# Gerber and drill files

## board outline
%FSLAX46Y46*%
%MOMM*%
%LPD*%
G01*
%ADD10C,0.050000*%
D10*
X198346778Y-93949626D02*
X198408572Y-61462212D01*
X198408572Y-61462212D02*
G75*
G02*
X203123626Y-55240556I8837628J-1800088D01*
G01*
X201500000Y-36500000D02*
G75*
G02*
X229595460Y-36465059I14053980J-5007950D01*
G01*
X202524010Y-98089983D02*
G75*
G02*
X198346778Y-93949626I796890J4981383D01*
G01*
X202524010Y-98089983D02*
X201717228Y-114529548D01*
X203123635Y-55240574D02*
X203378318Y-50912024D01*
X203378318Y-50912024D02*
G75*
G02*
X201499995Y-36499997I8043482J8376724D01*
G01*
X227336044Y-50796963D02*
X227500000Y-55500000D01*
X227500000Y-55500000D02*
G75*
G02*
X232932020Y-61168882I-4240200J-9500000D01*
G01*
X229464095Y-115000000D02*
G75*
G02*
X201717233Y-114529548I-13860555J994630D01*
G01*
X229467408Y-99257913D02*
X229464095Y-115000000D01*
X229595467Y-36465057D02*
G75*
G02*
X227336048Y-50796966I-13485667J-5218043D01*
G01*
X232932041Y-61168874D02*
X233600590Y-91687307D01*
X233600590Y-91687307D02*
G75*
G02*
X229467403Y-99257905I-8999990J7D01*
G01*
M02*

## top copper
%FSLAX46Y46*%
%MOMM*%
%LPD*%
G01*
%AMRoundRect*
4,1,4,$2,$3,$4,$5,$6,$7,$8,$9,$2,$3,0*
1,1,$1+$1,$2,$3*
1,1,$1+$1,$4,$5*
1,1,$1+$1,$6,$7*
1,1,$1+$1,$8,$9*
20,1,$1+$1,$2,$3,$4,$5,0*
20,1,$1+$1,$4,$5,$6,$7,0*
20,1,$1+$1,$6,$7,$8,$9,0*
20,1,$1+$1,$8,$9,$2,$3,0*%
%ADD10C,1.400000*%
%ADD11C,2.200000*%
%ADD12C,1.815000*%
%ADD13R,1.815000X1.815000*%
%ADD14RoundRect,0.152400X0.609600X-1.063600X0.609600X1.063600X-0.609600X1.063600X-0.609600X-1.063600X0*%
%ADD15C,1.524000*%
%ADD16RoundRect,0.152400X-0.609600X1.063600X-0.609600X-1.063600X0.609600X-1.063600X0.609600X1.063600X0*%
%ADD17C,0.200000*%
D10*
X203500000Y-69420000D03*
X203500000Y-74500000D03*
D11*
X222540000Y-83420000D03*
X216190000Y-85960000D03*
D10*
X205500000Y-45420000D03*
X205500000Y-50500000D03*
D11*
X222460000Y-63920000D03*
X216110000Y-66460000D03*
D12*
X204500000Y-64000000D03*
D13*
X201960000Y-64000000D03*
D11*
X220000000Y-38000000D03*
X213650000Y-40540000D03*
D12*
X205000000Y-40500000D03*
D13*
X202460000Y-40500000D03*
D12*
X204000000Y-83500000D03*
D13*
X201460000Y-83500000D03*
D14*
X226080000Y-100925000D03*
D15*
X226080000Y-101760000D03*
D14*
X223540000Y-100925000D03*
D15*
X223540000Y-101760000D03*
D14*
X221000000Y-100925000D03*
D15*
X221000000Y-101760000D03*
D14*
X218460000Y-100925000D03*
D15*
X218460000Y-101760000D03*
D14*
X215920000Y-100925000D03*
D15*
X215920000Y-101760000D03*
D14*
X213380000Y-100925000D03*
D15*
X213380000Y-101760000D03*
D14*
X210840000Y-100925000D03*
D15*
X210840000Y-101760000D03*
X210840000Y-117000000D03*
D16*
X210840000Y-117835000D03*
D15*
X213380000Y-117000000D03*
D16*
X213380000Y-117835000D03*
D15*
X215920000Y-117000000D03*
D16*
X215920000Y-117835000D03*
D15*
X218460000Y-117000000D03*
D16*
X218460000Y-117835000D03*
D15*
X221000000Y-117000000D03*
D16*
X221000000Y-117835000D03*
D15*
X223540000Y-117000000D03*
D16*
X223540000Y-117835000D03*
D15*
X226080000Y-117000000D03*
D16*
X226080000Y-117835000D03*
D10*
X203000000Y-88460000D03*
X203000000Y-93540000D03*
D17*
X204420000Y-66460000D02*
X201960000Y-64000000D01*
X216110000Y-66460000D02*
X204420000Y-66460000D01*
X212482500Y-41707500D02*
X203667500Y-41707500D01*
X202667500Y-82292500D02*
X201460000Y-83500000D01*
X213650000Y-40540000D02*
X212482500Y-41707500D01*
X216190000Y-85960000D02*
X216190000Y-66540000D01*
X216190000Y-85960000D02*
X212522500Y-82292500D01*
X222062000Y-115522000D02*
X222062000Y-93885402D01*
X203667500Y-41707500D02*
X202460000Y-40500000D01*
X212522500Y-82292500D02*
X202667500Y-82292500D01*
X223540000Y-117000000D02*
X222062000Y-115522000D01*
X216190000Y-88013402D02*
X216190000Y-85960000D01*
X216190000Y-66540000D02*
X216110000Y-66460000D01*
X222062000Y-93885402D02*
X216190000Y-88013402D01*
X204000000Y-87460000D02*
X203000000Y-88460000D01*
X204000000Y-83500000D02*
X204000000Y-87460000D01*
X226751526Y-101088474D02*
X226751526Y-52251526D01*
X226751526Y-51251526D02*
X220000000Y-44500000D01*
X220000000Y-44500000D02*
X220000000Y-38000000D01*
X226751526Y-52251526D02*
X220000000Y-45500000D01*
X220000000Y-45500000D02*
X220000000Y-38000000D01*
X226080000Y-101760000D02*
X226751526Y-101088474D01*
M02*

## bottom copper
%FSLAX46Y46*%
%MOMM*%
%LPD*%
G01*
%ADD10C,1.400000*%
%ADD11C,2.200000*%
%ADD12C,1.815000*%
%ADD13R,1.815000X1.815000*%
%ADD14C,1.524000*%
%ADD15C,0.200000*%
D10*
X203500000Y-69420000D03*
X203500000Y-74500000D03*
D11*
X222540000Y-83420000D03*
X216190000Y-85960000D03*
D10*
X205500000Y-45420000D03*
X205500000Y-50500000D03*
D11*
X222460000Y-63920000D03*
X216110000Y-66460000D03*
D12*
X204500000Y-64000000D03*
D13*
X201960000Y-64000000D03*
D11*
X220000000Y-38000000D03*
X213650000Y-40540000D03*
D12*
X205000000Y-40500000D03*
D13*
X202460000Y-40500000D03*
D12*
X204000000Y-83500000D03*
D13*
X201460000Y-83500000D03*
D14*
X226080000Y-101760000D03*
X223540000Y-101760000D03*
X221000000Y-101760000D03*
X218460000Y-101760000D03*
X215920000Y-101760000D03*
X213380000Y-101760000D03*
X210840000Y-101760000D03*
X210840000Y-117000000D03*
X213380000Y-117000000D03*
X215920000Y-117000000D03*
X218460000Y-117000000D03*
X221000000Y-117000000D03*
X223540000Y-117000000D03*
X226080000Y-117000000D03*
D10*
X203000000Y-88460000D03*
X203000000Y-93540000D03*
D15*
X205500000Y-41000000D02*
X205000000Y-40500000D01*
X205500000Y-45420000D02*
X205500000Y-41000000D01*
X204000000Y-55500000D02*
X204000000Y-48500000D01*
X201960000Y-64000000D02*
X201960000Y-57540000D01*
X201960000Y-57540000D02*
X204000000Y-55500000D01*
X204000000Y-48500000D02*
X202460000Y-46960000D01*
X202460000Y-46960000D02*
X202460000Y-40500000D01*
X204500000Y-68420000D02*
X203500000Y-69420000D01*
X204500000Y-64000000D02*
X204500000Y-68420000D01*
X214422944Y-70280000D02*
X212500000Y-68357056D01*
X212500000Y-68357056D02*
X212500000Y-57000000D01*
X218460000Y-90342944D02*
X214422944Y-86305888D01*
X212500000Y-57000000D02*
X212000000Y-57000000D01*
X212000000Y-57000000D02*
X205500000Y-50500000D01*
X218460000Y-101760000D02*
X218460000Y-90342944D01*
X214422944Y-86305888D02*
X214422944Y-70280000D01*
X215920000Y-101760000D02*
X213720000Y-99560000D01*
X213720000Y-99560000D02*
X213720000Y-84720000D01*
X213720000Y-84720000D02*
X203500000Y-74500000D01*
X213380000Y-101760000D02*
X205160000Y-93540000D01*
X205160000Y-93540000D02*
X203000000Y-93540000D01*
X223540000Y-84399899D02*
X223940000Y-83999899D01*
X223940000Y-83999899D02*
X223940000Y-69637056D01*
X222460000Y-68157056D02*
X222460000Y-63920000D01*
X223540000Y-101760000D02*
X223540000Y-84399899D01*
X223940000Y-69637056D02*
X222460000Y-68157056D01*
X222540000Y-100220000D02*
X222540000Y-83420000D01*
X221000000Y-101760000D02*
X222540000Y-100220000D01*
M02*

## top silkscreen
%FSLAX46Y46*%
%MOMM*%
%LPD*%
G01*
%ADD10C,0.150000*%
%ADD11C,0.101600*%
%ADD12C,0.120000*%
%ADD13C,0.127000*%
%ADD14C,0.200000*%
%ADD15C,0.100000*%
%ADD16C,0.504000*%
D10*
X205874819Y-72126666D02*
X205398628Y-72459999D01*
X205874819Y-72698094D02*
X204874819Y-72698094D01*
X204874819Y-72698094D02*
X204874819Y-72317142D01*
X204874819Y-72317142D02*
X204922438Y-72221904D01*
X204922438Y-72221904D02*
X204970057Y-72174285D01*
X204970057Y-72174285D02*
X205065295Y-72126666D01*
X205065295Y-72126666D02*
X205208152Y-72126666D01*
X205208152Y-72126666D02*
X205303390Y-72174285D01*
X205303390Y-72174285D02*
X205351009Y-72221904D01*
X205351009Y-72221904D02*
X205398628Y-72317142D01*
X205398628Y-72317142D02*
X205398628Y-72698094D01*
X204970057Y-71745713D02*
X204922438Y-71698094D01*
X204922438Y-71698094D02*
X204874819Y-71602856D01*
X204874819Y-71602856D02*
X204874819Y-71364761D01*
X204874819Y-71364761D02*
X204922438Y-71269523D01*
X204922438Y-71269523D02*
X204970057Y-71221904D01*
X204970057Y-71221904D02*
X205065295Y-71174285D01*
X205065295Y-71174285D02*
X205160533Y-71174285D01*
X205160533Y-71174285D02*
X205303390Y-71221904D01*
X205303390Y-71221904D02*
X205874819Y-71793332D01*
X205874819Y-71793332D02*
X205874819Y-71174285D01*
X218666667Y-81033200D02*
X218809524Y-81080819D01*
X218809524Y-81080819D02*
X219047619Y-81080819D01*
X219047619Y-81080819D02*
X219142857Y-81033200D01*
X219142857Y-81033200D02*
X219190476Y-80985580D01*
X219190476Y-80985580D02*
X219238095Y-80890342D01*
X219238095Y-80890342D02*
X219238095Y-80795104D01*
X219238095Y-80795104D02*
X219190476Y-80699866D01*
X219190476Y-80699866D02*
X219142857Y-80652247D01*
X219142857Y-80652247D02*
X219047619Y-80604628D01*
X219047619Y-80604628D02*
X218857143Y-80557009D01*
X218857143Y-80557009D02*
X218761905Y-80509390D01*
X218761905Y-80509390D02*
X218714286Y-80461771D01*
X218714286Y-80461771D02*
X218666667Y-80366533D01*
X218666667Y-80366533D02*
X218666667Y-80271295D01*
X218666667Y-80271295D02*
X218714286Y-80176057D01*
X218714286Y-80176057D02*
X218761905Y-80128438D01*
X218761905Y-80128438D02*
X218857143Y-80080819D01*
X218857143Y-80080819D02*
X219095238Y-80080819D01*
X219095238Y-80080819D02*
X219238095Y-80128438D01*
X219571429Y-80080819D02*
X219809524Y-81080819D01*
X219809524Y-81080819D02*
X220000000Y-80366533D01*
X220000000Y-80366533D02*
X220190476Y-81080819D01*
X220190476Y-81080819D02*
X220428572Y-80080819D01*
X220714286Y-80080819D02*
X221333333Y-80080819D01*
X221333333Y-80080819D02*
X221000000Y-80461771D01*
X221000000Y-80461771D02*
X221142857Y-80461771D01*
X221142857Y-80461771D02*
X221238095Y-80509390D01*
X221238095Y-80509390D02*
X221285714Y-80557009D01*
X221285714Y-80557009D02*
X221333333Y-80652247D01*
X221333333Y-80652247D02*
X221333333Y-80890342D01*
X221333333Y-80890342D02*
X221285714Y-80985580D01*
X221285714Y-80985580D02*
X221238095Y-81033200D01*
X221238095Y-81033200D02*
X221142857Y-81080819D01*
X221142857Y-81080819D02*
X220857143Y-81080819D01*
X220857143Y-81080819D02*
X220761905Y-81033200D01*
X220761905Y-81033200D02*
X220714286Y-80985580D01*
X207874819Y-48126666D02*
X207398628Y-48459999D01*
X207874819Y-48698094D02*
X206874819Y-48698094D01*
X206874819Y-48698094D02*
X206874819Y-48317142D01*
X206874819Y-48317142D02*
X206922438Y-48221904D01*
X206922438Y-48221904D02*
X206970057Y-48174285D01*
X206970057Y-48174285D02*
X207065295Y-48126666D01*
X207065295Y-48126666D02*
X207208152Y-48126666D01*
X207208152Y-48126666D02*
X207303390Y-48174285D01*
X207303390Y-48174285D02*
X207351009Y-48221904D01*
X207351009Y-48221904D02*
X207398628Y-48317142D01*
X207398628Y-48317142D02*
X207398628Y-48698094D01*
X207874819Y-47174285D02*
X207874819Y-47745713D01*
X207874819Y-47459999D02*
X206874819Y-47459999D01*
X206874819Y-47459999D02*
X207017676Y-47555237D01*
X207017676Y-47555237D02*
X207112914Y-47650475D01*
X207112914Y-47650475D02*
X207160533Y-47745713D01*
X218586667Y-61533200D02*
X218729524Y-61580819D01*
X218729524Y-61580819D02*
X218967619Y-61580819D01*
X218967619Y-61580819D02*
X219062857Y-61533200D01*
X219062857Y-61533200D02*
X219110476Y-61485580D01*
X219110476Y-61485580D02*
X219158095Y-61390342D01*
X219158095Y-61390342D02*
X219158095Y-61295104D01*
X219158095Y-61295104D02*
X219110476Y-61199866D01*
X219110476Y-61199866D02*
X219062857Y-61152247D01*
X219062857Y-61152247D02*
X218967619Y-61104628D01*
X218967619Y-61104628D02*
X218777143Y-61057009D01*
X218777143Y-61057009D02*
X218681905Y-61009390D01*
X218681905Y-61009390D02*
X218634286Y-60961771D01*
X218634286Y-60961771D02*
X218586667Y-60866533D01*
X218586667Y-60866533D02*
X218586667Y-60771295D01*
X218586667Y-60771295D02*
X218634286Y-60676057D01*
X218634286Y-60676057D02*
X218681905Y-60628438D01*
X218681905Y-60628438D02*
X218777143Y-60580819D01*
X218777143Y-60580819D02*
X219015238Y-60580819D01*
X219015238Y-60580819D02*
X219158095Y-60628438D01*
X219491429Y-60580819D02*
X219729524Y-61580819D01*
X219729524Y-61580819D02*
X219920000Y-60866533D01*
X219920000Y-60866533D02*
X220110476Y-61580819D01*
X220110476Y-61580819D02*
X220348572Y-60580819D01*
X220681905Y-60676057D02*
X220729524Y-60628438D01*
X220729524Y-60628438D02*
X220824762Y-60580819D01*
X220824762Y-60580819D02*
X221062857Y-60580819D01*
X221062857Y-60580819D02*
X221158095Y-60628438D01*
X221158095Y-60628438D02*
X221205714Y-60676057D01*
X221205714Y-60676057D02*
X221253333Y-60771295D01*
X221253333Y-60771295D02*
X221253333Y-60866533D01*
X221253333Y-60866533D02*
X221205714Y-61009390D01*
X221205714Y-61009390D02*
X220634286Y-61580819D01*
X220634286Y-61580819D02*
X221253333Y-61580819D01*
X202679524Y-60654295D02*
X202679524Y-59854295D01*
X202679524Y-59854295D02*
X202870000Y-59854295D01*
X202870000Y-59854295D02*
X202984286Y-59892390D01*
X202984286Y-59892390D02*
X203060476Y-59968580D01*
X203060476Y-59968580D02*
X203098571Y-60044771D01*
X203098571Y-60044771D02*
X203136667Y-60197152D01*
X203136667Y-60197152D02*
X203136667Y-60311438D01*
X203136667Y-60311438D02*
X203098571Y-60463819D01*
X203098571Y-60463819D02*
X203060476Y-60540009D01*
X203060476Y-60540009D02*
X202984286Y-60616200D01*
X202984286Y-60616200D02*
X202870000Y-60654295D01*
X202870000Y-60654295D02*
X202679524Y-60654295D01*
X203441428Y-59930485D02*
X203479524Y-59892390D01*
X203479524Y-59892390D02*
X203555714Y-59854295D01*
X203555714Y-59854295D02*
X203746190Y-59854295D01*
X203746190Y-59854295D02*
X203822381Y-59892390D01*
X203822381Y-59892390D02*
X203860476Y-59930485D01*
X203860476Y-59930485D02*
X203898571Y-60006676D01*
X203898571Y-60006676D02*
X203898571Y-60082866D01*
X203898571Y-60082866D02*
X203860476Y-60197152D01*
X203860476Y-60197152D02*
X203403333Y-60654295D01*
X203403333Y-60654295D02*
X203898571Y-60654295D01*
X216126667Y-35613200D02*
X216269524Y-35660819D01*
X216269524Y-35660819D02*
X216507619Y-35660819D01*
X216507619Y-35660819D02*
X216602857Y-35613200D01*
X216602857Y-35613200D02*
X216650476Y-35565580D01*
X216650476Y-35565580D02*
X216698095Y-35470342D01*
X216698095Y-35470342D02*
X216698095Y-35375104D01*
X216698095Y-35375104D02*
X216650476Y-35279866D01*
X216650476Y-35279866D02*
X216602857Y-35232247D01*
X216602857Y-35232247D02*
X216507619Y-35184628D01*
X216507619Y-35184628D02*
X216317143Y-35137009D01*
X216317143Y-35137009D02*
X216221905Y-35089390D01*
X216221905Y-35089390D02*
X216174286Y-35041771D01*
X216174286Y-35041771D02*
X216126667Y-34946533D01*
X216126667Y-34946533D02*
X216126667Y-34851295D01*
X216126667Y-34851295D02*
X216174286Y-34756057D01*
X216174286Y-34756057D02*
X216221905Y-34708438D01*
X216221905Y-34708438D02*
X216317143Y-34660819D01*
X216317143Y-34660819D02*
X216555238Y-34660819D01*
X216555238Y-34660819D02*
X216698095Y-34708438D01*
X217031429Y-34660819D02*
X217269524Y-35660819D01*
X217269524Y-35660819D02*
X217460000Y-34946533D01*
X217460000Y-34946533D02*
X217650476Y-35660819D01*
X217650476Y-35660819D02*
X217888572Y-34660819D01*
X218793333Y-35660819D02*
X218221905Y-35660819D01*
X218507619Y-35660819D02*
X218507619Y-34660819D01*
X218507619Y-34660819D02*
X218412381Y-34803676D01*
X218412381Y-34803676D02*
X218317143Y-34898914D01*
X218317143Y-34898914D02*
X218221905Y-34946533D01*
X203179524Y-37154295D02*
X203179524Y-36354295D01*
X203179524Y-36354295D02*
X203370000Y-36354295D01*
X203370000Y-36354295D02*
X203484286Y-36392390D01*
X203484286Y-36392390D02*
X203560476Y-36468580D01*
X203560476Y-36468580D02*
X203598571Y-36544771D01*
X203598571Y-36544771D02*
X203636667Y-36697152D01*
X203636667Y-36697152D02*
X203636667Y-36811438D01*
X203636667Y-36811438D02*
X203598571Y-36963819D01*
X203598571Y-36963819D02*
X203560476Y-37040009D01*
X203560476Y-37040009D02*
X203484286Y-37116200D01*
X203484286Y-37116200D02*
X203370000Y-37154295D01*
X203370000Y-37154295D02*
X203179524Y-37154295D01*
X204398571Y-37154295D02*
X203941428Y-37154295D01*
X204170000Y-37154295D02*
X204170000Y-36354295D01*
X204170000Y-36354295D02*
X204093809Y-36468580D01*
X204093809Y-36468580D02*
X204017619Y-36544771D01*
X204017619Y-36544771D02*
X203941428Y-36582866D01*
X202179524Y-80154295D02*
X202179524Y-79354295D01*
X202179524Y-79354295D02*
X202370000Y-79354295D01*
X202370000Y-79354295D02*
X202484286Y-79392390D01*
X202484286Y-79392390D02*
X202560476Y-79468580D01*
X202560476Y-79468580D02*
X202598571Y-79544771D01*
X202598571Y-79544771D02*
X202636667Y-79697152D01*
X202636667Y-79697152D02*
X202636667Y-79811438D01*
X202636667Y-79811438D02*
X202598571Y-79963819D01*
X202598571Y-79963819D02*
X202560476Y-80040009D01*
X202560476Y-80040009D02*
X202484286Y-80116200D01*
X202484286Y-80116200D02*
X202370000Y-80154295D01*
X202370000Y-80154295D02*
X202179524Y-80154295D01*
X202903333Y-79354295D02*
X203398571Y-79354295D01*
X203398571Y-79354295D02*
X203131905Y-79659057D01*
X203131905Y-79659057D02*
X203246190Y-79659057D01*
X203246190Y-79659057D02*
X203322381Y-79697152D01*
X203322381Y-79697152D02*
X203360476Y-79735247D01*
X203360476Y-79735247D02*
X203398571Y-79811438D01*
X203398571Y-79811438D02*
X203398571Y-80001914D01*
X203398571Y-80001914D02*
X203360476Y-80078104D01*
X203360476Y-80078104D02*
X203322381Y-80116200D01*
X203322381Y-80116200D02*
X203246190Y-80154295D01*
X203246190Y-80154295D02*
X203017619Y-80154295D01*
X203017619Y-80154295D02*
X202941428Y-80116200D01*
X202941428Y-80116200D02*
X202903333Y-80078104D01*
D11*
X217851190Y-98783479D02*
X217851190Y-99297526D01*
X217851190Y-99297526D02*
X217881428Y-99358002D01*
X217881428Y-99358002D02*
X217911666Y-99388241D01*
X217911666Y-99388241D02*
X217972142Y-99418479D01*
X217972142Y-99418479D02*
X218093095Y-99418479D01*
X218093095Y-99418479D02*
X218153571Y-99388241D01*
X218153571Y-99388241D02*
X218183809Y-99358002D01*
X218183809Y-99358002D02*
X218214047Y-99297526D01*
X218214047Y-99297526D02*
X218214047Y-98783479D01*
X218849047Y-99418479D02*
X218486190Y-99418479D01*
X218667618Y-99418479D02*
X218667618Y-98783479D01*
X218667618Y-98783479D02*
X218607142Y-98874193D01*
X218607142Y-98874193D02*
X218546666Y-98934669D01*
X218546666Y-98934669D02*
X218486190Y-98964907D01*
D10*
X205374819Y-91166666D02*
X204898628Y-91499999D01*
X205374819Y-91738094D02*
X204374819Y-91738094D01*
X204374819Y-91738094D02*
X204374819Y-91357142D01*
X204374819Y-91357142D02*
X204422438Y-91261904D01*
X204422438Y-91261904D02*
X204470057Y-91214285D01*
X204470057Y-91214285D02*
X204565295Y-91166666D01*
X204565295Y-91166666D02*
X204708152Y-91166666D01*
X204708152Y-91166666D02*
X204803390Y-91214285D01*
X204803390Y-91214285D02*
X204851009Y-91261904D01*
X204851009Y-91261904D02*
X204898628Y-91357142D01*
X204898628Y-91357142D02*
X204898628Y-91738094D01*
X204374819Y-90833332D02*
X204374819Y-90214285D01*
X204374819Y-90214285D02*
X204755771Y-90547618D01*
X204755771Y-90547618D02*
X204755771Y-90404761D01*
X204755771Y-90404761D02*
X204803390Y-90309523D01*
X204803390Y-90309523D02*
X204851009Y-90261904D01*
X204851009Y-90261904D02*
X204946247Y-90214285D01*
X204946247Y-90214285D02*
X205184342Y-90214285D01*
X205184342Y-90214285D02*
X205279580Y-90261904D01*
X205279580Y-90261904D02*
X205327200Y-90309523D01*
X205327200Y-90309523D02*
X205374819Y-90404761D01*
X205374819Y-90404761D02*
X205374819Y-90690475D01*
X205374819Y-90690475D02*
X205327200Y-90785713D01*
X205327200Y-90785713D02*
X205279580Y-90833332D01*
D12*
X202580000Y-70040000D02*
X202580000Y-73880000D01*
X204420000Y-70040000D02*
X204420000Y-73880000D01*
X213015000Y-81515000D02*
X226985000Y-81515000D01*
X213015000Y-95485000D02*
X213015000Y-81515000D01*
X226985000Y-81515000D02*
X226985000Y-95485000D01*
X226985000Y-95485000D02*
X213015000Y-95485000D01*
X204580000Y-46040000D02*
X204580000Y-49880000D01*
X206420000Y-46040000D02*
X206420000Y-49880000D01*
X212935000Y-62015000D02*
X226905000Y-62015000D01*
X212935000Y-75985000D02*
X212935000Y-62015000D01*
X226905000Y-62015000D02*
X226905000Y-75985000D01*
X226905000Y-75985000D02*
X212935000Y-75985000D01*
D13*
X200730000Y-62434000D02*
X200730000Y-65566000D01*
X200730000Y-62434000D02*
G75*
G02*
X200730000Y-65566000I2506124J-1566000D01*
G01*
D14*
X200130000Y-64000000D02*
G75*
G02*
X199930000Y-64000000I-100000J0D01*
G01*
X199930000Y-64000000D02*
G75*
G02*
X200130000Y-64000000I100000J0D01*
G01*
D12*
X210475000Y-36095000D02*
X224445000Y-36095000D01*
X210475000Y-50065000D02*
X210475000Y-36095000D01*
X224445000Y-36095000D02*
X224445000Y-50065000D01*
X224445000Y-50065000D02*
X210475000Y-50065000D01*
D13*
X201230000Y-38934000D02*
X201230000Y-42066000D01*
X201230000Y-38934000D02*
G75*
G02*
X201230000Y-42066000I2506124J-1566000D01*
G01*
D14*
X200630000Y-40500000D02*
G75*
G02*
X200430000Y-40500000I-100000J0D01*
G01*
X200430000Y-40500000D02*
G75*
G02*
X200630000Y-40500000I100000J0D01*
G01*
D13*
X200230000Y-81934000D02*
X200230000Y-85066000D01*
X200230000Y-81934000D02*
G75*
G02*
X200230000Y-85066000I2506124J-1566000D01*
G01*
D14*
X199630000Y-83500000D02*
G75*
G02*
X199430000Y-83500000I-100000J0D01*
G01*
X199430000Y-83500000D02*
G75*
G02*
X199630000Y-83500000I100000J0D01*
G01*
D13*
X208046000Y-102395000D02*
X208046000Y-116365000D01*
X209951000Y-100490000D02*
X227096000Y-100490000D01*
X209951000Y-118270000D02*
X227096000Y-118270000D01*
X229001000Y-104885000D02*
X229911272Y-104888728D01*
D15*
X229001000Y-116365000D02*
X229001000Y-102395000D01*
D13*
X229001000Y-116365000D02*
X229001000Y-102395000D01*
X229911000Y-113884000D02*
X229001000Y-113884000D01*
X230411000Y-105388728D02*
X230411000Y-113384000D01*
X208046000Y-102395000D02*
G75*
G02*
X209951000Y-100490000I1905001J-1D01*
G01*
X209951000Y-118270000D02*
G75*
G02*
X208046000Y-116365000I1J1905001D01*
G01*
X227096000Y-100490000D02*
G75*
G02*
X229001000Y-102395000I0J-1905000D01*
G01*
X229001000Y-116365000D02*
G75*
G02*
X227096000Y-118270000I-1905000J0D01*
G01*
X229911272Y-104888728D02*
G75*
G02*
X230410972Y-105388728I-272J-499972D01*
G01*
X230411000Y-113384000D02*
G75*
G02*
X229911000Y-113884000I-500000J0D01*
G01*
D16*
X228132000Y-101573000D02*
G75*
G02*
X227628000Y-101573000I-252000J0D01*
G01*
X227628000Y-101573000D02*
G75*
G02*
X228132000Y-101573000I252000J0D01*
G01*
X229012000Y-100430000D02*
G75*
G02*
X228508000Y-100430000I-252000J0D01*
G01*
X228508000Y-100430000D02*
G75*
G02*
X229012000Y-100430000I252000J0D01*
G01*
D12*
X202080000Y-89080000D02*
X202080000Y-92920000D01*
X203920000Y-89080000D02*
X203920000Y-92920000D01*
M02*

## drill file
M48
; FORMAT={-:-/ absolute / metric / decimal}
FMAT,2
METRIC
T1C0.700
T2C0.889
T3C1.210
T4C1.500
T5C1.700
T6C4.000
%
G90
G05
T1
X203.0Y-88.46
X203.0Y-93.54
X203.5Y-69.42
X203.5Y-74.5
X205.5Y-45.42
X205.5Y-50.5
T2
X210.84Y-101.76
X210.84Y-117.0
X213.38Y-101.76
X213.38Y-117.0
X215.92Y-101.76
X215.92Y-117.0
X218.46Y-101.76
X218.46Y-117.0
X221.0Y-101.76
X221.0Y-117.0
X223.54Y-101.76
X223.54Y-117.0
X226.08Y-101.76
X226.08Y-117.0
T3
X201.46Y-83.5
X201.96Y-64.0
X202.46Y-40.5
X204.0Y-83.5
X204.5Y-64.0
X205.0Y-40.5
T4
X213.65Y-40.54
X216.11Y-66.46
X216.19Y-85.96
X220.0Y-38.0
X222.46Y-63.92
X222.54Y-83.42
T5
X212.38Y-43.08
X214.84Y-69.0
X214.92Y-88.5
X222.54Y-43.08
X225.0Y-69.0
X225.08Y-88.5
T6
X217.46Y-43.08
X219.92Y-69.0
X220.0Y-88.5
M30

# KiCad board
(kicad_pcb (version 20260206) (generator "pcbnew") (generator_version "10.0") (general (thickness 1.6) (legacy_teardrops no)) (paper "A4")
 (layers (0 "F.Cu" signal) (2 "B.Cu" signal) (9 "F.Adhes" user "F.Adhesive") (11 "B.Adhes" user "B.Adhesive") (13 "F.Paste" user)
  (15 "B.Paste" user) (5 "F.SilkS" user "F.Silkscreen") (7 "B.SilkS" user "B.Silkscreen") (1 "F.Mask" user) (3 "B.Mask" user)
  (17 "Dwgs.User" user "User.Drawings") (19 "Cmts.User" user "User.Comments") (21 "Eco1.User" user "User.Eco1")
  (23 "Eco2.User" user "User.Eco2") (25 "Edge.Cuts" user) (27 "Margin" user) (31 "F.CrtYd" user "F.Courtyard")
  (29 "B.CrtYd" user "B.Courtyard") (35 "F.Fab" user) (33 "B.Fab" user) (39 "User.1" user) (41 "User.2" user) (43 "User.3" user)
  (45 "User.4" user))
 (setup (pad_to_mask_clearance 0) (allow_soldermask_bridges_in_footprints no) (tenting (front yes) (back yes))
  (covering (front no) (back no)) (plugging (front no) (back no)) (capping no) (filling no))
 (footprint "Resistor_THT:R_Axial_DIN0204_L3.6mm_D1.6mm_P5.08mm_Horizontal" (layer "F.Cu") (at 203.5 69.42 -90)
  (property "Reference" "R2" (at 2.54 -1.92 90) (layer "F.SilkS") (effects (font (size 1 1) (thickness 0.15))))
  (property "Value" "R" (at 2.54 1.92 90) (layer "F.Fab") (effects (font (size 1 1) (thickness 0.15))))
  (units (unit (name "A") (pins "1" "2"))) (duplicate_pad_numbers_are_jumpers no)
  (fp_line (start 0.62 0.92) (end 4.46 0.92) (stroke (width 0.12) (type solid)) (layer "F.SilkS"))
  (fp_line (start 0.62 -0.92) (end 4.46 -0.92) (stroke (width 0.12) (type solid)) (layer "F.SilkS"))
  (pad "1" thru_hole circle (at 0 0 270) (size 1.4 1.4) (drill 0.7) (layers "*.Cu" "*.Mask") (remove_unused_layers no) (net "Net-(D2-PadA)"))
  (pad "2" thru_hole circle (at 5.08 0 270) (size 1.4 1.4) (drill 0.7) (layers "*.Cu" "*.Mask") (remove_unused_layers no) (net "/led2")))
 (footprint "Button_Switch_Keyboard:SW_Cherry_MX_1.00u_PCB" (layer "F.Cu") (at 222.54 83.42)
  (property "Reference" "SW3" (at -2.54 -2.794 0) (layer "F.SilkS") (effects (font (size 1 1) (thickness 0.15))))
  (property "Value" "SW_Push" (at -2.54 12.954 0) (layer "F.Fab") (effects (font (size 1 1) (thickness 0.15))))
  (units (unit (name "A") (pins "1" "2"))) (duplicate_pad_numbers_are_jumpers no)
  (fp_line (start -9.525 -1.905) (end 4.445 -1.905) (stroke (width 0.12) (type solid)) (layer "F.SilkS"))
  (fp_line (start -9.525 12.065) (end -9.525 -1.905) (stroke (width 0.12) (type solid)) (layer "F.SilkS"))
  (fp_line (start 4.445 -1.905) (end 4.445 12.065) (stroke (width 0.12) (type solid)) (layer "F.SilkS"))
  (fp_line (start 4.445 12.065) (end -9.525 12.065) (stroke (width 0.12) (type solid)) (layer "F.SilkS"))
  (pad "" np_thru_hole circle (at -7.62 5.08) (size 1.7 1.7) (drill 1.7) (layers "*.Cu" "*.Mask"))
  (pad "" np_thru_hole circle (at -2.54 5.08) (size 4 4) (drill 4) (layers "*.Cu" "*.Mask"))
  (pad "" np_thru_hole circle (at 2.54 5.08) (size 1.7 1.7) (drill 1.7) (layers "*.Cu" "*.Mask"))
  (pad "1" thru_hole circle (at 0 0) (size 2.2 2.2) (drill 1.5) (layers "*.Cu" "*.Mask") (remove_unused_layers no) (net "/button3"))
  (pad "2" thru_hole circle (at -6.35 2.54) (size 2.2 2.2) (drill 1.5) (layers "*.Cu" "*.Mask") (remove_unused_layers no) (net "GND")))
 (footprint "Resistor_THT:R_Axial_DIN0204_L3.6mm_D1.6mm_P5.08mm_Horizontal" (layer "F.Cu") (at 205.5 45.42 -90)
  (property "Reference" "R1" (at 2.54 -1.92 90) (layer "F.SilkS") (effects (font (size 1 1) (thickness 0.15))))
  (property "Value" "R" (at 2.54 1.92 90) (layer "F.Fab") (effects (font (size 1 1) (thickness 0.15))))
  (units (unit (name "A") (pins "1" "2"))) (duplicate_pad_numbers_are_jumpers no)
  (fp_line (start 0.62 0.92) (end 4.46 0.92) (stroke (width 0.12) (type solid)) (layer "F.SilkS"))
  (fp_line (start 0.62 -0.92) (end 4.46 -0.92) (stroke (width 0.12) (type solid)) (layer "F.SilkS"))
  (pad "1" thru_hole circle (at 0 0 270) (size 1.4 1.4) (drill 0.7) (layers "*.Cu" "*.Mask") (remove_unused_layers no) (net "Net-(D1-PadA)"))
  (pad "2" thru_hole circle (at 5.08 0 270) (size 1.4 1.4) (drill 0.7) (layers "*.Cu" "*.Mask") (remove_unused_layers no) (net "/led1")))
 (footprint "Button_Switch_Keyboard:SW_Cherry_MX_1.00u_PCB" (layer "F.Cu") (at 222.46 63.92)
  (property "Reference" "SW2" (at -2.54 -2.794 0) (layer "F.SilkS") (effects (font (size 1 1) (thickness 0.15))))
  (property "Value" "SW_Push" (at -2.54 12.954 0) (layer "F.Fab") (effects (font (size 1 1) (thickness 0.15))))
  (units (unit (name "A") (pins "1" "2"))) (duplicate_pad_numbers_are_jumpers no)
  (fp_line (start -9.525 -1.905) (end 4.445 -1.905) (stroke (width 0.12) (type solid)) (layer "F.SilkS"))
  (fp_line (start -9.525 12.065) (end -9.525 -1.905) (stroke (width 0.12) (type solid)) (layer "F.SilkS"))
  (fp_line (start 4.445 -1.905) (end 4.445 12.065) (stroke (width 0.12) (type solid)) (layer "F.SilkS"))
  (fp_line (start 4.445 12.065) (end -9.525 12.065) (stroke (width 0.12) (type solid)) (layer "F.SilkS"))
  (pad "" np_thru_hole circle (at -7.62 5.08) (size 1.7 1.7) (drill 1.7) (layers "*.Cu" "*.Mask"))
  (pad "" np_thru_hole circle (at -2.54 5.08) (size 4 4) (drill 4) (layers "*.Cu" "*.Mask"))
  (pad "" np_thru_hole circle (at 2.54 5.08) (size 1.7 1.7) (drill 1.7) (layers "*.Cu" "*.Mask"))
  (pad "1" thru_hole circle (at 0 0) (size 2.2 2.2) (drill 1.5) (layers "*.Cu" "*.Mask") (remove_unused_layers no) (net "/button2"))
  (pad "2" thru_hole circle (at -6.35 2.54) (size 2.2 2.2) (drill 1.5) (layers "*.Cu" "*.Mask") (remove_unused_layers no) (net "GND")))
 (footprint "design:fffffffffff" (layer "F.Cu") (at 215 35 180)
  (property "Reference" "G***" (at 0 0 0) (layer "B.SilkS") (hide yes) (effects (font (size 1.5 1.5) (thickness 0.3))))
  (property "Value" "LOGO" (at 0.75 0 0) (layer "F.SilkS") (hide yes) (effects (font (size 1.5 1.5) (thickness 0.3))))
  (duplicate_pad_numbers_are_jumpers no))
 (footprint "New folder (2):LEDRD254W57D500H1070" (layer "F.Cu") (at 203.23 64)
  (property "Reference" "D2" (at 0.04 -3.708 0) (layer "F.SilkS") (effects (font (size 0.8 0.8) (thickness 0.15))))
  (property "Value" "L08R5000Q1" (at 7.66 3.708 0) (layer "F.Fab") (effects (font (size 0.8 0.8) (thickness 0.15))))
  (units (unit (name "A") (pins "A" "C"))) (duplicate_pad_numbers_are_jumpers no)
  (fp_line (start -2.5 -1.566) (end -2.5 1.566) (stroke (width 0.127) (type solid)) (layer "F.SilkS"))
  (fp_arc (start -2.5 -1.566) (mid 2.961291 0) (end -2.5 1.566) (stroke (width 0.127) (type solid)) (layer "F.SilkS"))
  (fp_circle (center -3.2 0) (end -3.1 0) (stroke (width 0.2) (type solid)) (fill no) (layer "F.SilkS"))
  (pad "A" thru_hole circle (at 1.27 0) (size 1.815 1.815) (drill 1.21) (layers "*.Cu" "*.Mask") (remove_unused_layers no)
   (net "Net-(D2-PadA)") (solder_mask_margin 0.102))
  (pad "C" thru_hole rect (at -1.27 0) (size 1.815 1.815) (drill 1.21) (layers "*.Cu" "*.Mask") (remove_unused_layers no) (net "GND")
   (solder_mask_margin 0.102)))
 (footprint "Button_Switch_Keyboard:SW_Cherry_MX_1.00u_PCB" (layer "F.Cu") (at 220 38)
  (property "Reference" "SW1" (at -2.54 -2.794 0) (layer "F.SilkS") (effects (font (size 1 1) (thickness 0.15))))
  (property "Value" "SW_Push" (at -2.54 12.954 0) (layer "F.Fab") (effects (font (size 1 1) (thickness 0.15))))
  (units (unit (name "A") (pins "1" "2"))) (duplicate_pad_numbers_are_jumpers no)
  (fp_line (start -9.525 -1.905) (end 4.445 -1.905) (stroke (width 0.12) (type solid)) (layer "F.SilkS"))
  (fp_line (start -9.525 12.065) (end -9.525 -1.905) (stroke (width 0.12) (type solid)) (layer "F.SilkS"))
  (fp_line (start 4.445 -1.905) (end 4.445 12.065) (stroke (width 0.12) (type solid)) (layer "F.SilkS"))
  (fp_line (start 4.445 12.065) (end -9.525 12.065) (stroke (width 0.12) (type solid)) (layer "F.SilkS"))
  (pad "" np_thru_hole circle (at -7.62 5.08) (size 1.7 1.7) (drill 1.7) (layers "*.Cu" "*.Mask"))
  (pad "" np_thru_hole circle (at -2.54 5.08) (size 4 4) (drill 4) (layers "*.Cu" "*.Mask"))
  (pad "" np_thru_hole circle (at 2.54 5.08) (size 1.7 1.7) (drill 1.7) (layers "*.Cu" "*.Mask"))
  (pad "1" thru_hole circle (at 0 0) (size 2.2 2.2) (drill 1.5) (layers "*.Cu" "*.Mask") (remove_unused_layers no) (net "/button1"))
  (pad "2" thru_hole circle (at -6.35 2.54) (size 2.2 2.2) (drill 1.5) (layers "*.Cu" "*.Mask") (remove_unused_layers no) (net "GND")))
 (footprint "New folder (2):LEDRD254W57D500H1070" (layer "F.Cu") (at 203.73 40.5)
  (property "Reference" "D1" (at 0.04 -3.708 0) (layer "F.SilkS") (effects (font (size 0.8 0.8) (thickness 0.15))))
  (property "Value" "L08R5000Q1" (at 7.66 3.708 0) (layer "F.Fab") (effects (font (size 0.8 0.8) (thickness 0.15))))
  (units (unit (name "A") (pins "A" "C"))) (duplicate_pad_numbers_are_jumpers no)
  (fp_line (start -2.5 -1.566) (end -2.5 1.566) (stroke (width 0.127) (type solid)) (layer "F.SilkS"))
  (fp_arc (start -2.5 -1.566) (mid 2.961291 0) (end -2.5 1.566) (stroke (width 0.127) (type solid)) (layer "F.SilkS"))
  (fp_circle (center -3.2 0) (end -3.1 0) (stroke (width 0.2) (type solid)) (fill no) (layer "F.SilkS"))
  (pad "A" thru_hole circle (at 1.27 0) (size 1.815 1.815) (drill 1.21) (layers "*.Cu" "*.Mask") (remove_unused_layers no)
   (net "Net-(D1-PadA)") (solder_mask_margin 0.102))
  (pad "C" thru_hole rect (at -1.27 0) (size 1.815 1.815) (drill 1.21) (layers "*.Cu" "*.Mask") (remove_unused_layers no) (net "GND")
   (solder_mask_margin 0.102)))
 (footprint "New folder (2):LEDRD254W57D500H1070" (layer "F.Cu") (at 202.73 83.5)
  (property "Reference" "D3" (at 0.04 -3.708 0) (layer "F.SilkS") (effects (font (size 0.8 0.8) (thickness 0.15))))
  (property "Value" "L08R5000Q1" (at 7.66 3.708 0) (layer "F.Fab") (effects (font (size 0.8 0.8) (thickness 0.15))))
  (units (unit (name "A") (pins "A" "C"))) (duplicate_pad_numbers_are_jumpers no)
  (fp_line (start -2.5 -1.566) (end -2.5 1.566) (stroke (width 0.127) (type solid)) (layer "F.SilkS"))
  (fp_arc (start -2.5 -1.566) (mid 2.961291 0) (end -2.5 1.566) (stroke (width 0.127) (type solid)) (layer "F.SilkS"))
  (fp_circle (center -3.2 0) (end -3.1 0) (stroke (width 0.2) (type solid)) (fill no) (layer "F.SilkS"))
  (pad "A" thru_hole circle (at 1.27 0) (size 1.815 1.815) (drill 1.21) (layers "*.Cu" "*.Mask") (remove_unused_layers no)
   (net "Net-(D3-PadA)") (solder_mask_margin 0.102))
  (pad "C" thru_hole rect (at -1.27 0) (size 1.815 1.815) (drill 1.21) (layers "*.Cu" "*.Mask") (remove_unused_layers no) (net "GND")
   (solder_mask_margin 0.102)))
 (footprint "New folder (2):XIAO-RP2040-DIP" (layer "F.Cu") (at 218.46 109.38)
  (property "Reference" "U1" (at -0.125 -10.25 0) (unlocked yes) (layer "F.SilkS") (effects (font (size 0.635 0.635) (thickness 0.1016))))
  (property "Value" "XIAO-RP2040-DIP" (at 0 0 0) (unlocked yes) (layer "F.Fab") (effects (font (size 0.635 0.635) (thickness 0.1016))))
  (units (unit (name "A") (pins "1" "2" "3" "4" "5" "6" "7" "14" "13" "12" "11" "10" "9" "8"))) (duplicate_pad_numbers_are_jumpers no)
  (fp_line (start -10.414 -6.985) (end -10.414 6.985) (stroke (width 0.127) (type solid)) (layer "F.SilkS"))
  (fp_line (start -8.509 -8.89) (end 8.636 -8.89) (stroke (width 0.127) (type solid)) (layer "F.SilkS"))
  (fp_line (start -8.509 8.89) (end 8.636 8.89) (stroke (width 0.127) (type solid)) (layer "F.SilkS"))
  (fp_line (start 10.541 -4.495) (end 11.451272 -4.491272) (stroke (width 0.127) (type solid)) (layer "F.SilkS"))
  (fp_line (start 10.541 6.985) (end 10.541 -6.985) (stroke (width 0.1) (type solid)) (layer "F.SilkS"))
  (fp_line (start 10.541 6.985) (end 10.541 -6.985) (stroke (width 0.127) (type solid)) (layer "F.SilkS"))
  (fp_line (start 11.451 4.504) (end 10.541 4.504) (stroke (width 0.127) (type solid)) (layer "F.SilkS"))
  (fp_line (start 11.951 -3.991272) (end 11.951 4.004) (stroke (width 0.127) (type solid)) (layer "F.SilkS"))
  (fp_arc (start -10.414 -6.985) (mid -9.856038 -8.332038) (end -8.509 -8.89) (stroke (width 0.127) (type solid)) (layer "F.SilkS"))
  (fp_arc (start -8.509 8.89) (mid -9.856038 8.332038) (end -10.414 6.985) (stroke (width 0.127) (type solid)) (layer "F.SilkS"))
  (fp_arc (start 8.636 -8.89) (mid 9.983038 -8.332038) (end 10.541 -6.985) (stroke (width 0.127) (type solid)) (layer "F.SilkS"))
  (fp_arc (start 10.541 6.985) (mid 9.983038 8.332038) (end 8.636 8.89) (stroke (width 0.127) (type solid)) (layer "F.SilkS"))
  (fp_arc (start 11.451272 -4.491272) (mid 11.804644 -4.344724) (end 11.951 -3.991272) (stroke (width 0.127) (type default))
   (layer "F.SilkS"))
  (fp_arc (start 11.951 4.004) (mid 11.804553 4.357553) (end 11.451 4.504) (stroke (width 0.127) (type default)) (layer "F.SilkS"))
  (fp_circle (center 9.42 -7.807) (end 9.674 -7.807) (stroke (width 0.5) (type solid)) (fill yes) (layer "F.SilkS"))
  (fp_circle (center 10.3 -8.95) (end 10.554 -8.95) (stroke (width 0.5) (type solid)) (fill yes) (layer "F.SilkS"))
  (pad "1" smd roundrect (at 7.62 -8.455 90) (size 2.432 1.524) (layers "F.Cu" "F.Mask") (roundrect_rratio 0.1) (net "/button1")
   (thermal_bridge_angle 45))
  (pad "1" thru_hole circle (at 7.62 -7.62 90) (size 1.524 1.524) (drill 0.889) (layers "*.Cu" "*.Mask") (remove_unused_layers no)
   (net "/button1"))
  (pad "2" smd roundrect (at 5.08 -8.455 90) (size 2.432 1.524) (layers "F.Cu" "F.Mask") (roundrect_rratio 0.1) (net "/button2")
   (thermal_bridge_angle 45))
  (pad "2" thru_hole circle (at 5.08 -7.62 90) (size 1.524 1.524) (drill 0.889) (layers "*.Cu" "*.Mask") (remove_unused_layers no)
   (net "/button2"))
  (pad "3" smd roundrect (at 2.54 -8.455 90) (size 2.432 1.524) (layers "F.Cu" "F.Mask") (roundrect_rratio 0.1) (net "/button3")
   (thermal_bridge_angle 45))
  (pad "3" thru_hole circle (at 2.54 -7.62 90) (size 1.524 1.524) (drill 0.889) (layers "*.Cu" "*.Mask") (remove_unused_layers no)
   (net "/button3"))
  (pad "4" smd roundrect (at 0 -8.455 90) (size 2.432 1.524) (layers "F.Cu" "F.Mask") (roundrect_rratio 0.1) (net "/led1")
   (thermal_bridge_angle 45))
  (pad "4" thru_hole circle (at 0 -7.62 90) (size 1.524 1.524) (drill 0.889) (layers "*.Cu" "*.Mask") (remove_unused_layers no)
   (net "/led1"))
  (pad "5" smd roundrect (at -2.54 -8.455 90) (size 2.432 1.524) (layers "F.Cu" "F.Mask") (roundrect_rratio 0.1) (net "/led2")
   (thermal_bridge_angle 45))
  (pad "5" thru_hole circle (at -2.54 -7.62 90) (size 1.524 1.524) (drill 0.889) (layers "*.Cu" "*.Mask") (remove_unused_layers no)
   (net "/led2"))
  (pad "6" smd roundrect (at -5.08 -8.455 90) (size 2.432 1.524) (layers "F.Cu" "F.Mask") (roundrect_rratio 0.1) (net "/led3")
   (thermal_bridge_angle 45))
  (pad "6" thru_hole circle (at -5.08 -7.62 90) (size 1.524 1.524) (drill 0.889) (layers "*.Cu" "*.Mask") (remove_unused_layers no)
   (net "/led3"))
  (pad "7" smd roundrect (at -7.62 -8.455 90) (size 2.432 1.524) (layers "F.Cu" "F.Mask") (roundrect_rratio 0.1)
   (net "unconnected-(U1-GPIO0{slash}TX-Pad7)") (thermal_bridge_angle 45))
  (pad "7" thru_hole circle (at -7.62 -7.62 90) (size 1.524 1.524) (drill 0.889) (layers "*.Cu" "*.Mask") (remove_unused_layers no)
   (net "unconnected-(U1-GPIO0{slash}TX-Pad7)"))
  (pad "8" thru_hole circle (at -7.62 7.62 270) (size 1.524 1.524) (drill 0.889) (layers "*.Cu" "*.Mask") (remove_unused_layers no)
   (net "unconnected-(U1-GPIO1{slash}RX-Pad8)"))
  (pad "8" smd roundrect (at -7.62 8.455 270) (size 2.432 1.524) (layers "F.Cu" "F.Mask") (roundrect_rratio 0.1)
   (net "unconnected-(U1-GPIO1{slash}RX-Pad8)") (thermal_bridge_angle 45))
  (pad "9" thru_hole circle (at -5.08 7.62 270) (size 1.524 1.524) (drill 0.889) (layers "*.Cu" "*.Mask") (remove_unused_layers no)
   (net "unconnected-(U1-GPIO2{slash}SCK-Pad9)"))
  (pad "9" smd roundrect (at -5.08 8.455 270) (size 2.432 1.524) (layers "F.Cu" "F.Mask") (roundrect_rratio 0.1)
   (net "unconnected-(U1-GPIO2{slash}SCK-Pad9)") (thermal_bridge_angle 45))
  (pad "10" thru_hole circle (at -2.54 7.62 270) (size 1.524 1.524) (drill 0.889) (layers "*.Cu" "*.Mask") (remove_unused_layers no)
   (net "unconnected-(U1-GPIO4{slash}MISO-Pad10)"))
  (pad "10" smd roundrect (at -2.54 8.455 270) (size 2.432 1.524) (layers "F.Cu" "F.Mask") (roundrect_rratio 0.1)
   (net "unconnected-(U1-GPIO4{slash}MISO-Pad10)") (thermal_bridge_angle 45))
  (pad "11" thru_hole circle (at 0 7.62 270) (size 1.524 1.524) (drill 0.889) (layers "*.Cu" "*.Mask") (remove_unused_layers no)
   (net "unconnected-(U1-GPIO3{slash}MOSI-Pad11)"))
  (pad "11" smd roundrect (at 0 8.455 270) (size 2.432 1.524) (layers "F.Cu" "F.Mask") (roundrect_rratio 0.1)
   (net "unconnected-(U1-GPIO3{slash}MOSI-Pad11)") (thermal_bridge_angle 45))
  (pad "12" thru_hole circle (at 2.54 7.62 270) (size 1.524 1.524) (drill 0.889) (layers "*.Cu" "*.Mask") (remove_unused_layers no)
   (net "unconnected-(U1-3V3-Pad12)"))
  (pad "12" smd roundrect (at 2.54 8.455 270) (size 2.432 1.524) (layers "F.Cu" "F.Mask") (roundrect_rratio 0.1)
   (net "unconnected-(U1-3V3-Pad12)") (thermal_bridge_angle 45))
  (pad "13" thru_hole circle (at 5.08 7.62 270) (size 1.524 1.524) (drill 0.889) (layers "*.Cu" "*.Mask") (remove_unused_layers no)
   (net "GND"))
  (pad "13" smd roundrect (at 5.08 8.455 270) (size 2.432 1.524) (layers "F.Cu" "F.Mask") (roundrect_rratio 0.1) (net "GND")
   (thermal_bridge_angle 45))
  (pad "14" thru_hole circle (at 7.62 7.62 270) (size 1.524 1.524) (drill 0.889) (layers "*.Cu" "*.Mask") (remove_unused_layers no)
   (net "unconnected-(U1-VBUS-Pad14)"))
  (pad "14" smd roundrect (at 7.62 8.455 270) (size 2.432 1.524) (layers "F.Cu" "F.Mask") (roundrect_rratio 0.1)
   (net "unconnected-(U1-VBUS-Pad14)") (thermal_bridge_angle 45)))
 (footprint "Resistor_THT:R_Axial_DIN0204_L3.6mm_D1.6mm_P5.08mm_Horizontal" (layer "F.Cu") (at 203 88.46 -90)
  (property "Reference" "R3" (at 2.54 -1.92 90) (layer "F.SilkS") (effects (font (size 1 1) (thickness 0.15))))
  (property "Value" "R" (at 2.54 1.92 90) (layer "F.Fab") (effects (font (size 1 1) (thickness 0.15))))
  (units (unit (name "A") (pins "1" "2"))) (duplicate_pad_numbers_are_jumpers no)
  (fp_line (start 0.62 0.92) (end 4.46 0.92) (stroke (width 0.12) (type solid)) (layer "F.SilkS"))
  (fp_line (start 0.62 -0.92) (end 4.46 -0.92) (stroke (width 0.12) (type solid)) (layer "F.SilkS"))
  (pad "1" thru_hole circle (at 0 0 270) (size 1.4 1.4) (drill 0.7) (layers "*.Cu" "*.Mask") (remove_unused_layers no) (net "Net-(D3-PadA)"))
  (pad "2" thru_hole circle (at 5.08 0 270) (size 1.4 1.4) (drill 0.7) (layers "*.Cu" "*.Mask") (remove_unused_layers no) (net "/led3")))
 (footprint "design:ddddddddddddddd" (layer "F.Cu") (at 216 84.5)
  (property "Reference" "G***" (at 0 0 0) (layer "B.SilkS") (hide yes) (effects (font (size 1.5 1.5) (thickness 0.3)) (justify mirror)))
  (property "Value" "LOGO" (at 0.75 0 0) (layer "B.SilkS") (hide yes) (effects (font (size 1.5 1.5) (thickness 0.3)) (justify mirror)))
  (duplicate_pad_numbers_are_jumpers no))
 (gr_line (start 198.346778 93.949626) (end 198.408572 61.462212) (stroke (width 0.05) (type solid)) (layer "Edge.Cuts"))
 (gr_arc (start 198.408572 61.462212) (mid 200.058094 57.814829) (end 203.123635 55.240574) (stroke (width 0.05) (type default))
  (layer "Edge.Cuts"))
 (gr_arc (start 201.5 36.5) (mid 215.570982 26.588375) (end 229.595467 36.465057) (stroke (width 0.05) (type default)) (layer "Edge.Cuts"))
 (gr_arc (start 202.52401 98.089983) (mid 199.769593 96.691536) (end 198.346778 93.949626) (stroke (width 0.05) (type default))
  (layer "Edge.Cuts"))
 (gr_line (start 202.52401 98.089983) (end 201.717228 114.529548) (stroke (width 0.05) (type default)) (layer "Edge.Cuts"))
 (gr_line (start 203.123635 55.240574) (end 203.378318 50.912024) (stroke (width 0.05) (type default)) (layer "Edge.Cuts"))
 (gr_arc (start 203.378318 50.912024) (mid 199.905969 44.036162) (end 201.5 36.5) (stroke (width 0.05) (type default)) (layer "Edge.Cuts"))
 (gr_line (start 227.336044 50.796963) (end 227.5 55.5) (stroke (width 0.05) (type default)) (layer "Edge.Cuts"))
 (gr_arc (start 227.5 55.5) (mid 230.77133 57.802327) (end 232.932041 61.168874) (stroke (width 0.05) (type default)) (layer "Edge.Cuts"))
 (gr_arc (start 229.464095 115) (mid 215.367959 127.899572) (end 201.717228 114.529548) (stroke (width 0.05) (type default))
  (layer "Edge.Cuts"))
 (gr_line (start 229.467408 99.257913) (end 229.464095 115) (stroke (width 0.05) (type solid)) (layer "Edge.Cuts"))
 (gr_arc (start 229.595467 36.465057) (mid 230.391429 43.947172) (end 227.336044 50.796963) (stroke (width 0.05) (type default))
  (layer "Edge.Cuts"))
 (gr_line (start 232.932041 61.168874) (end 233.60059 91.687307) (stroke (width 0.05) (type default)) (layer "Edge.Cuts"))
 (gr_arc (start 233.60059 91.687307) (mid 232.5 96) (end 229.467408 99.257913) (stroke (width 0.05) (type default)) (layer "Edge.Cuts"))
 (segment (start 205.5 41) (end 205 40.5) (width 0.2) (layer "B.Cu") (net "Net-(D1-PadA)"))
 (segment (start 205.5 45.42) (end 205.5 41) (width 0.2) (layer "B.Cu") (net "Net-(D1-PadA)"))
 (segment (start 204.42 66.46) (end 201.96 64) (width 0.2) (layer "F.Cu") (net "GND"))
 (segment (start 216.11 66.46) (end 204.42 66.46) (width 0.2) (layer "F.Cu") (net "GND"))
 (segment (start 212.4825 41.7075) (end 203.6675 41.7075) (width 0.2) (layer "F.Cu") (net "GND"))
 (segment (start 202.6675 82.2925) (end 201.46 83.5) (width 0.2) (layer "F.Cu") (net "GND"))
 (segment (start 213.65 40.54) (end 212.4825 41.7075) (width 0.2) (layer "F.Cu") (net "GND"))
 (segment (start 216.19 85.96) (end 216.19 66.54) (width 0.2) (layer "F.Cu") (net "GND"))
 (segment (start 216.19 85.96) (end 212.5225 82.2925) (width 0.2) (layer "F.Cu") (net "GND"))
 (segment (start 222.062 115.522) (end 222.062 93.885402) (width 0.2) (layer "F.Cu") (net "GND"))
 (segment (start 203.6675 41.7075) (end 202.46 40.5) (width 0.2) (layer "F.Cu") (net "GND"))
 (segment (start 212.5225 82.2925) (end 202.6675 82.2925) (width 0.2) (layer "F.Cu") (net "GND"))
 (segment (start 223.54 117) (end 222.062 115.522) (width 0.2) (layer "F.Cu") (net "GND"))
 (segment (start 216.19 88.013402) (end 216.19 85.96) (width 0.2) (layer "F.Cu") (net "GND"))
 (segment (start 216.19 66.54) (end 216.11 66.46) (width 0.2) (layer "F.Cu") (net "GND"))
 (segment (start 222.062 93.885402) (end 216.19 88.013402) (width 0.2) (layer "F.Cu") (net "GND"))
 (segment (start 204 55.5) (end 204 48.5) (width 0.2) (layer "B.Cu") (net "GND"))
 (segment (start 201.96 64) (end 201.96 57.54) (width 0.2) (layer "B.Cu") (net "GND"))
 (segment (start 201.96 57.54) (end 204 55.5) (width 0.2) (layer "B.Cu") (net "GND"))
 (segment (start 204 48.5) (end 202.46 46.96) (width 0.2) (layer "B.Cu") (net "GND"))
 (segment (start 202.46 46.96) (end 202.46 40.5) (width 0.2) (layer "B.Cu") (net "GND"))
 (segment (start 204.5 68.42) (end 203.5 69.42) (width 0.2) (layer "B.Cu") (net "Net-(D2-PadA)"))
 (segment (start 204.5 64) (end 204.5 68.42) (width 0.2) (layer "B.Cu") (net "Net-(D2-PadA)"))
 (segment (start 204 87.46) (end 203 88.46) (width 0.2) (layer "F.Cu") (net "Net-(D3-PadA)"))
 (segment (start 204 83.5) (end 204 87.46) (width 0.2) (layer "F.Cu") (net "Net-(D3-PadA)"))
 (segment (start 214.422944 70.28) (end 212.5 68.357056) (width 0.2) (layer "B.Cu") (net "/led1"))
 (segment (start 212.5 68.357056) (end 212.5 57) (width 0.2) (layer "B.Cu") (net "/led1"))
 (segment (start 218.46 90.342944) (end 214.422944 86.305888) (width 0.2) (layer "B.Cu") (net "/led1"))
 (segment (start 212.5 57) (end 212 57) (width 0.2) (layer "B.Cu") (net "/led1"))
 (segment (start 212 57) (end 205.5 50.5) (width 0.2) (layer "B.Cu") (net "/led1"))
 (segment (start 218.46 101.76) (end 218.46 90.342944) (width 0.2) (layer "B.Cu") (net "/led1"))
 (segment (start 214.422944 86.305888) (end 214.422944 70.28) (width 0.2) (layer "B.Cu") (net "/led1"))
 (segment (start 215.92 101.76) (end 213.72 99.56) (width 0.2) (layer "B.Cu") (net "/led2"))
 (segment (start 213.72 99.56) (end 213.72 84.72) (width 0.2) (layer "B.Cu") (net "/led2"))
 (segment (start 213.72 84.72) (end 203.5 74.5) (width 0.2) (layer "B.Cu") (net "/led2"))
 (segment (start 213.38 101.76) (end 205.16 93.54) (width 0.2) (layer "B.Cu") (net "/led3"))
 (segment (start 205.16 93.54) (end 203 93.54) (width 0.2) (layer "B.Cu") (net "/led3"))
 (segment (start 226.751526 101.088474) (end 226.751526 52.251526) (width 0.2) (layer "F.Cu") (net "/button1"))
 (segment (start 226.751526 51.251526) (end 220 44.5) (width 0.2) (layer "F.Cu") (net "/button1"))
 (segment (start 220 44.5) (end 220 38) (width 0.2) (layer "F.Cu") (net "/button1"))
 (segment (start 226.751526 52.251526) (end 220 45.5) (width 0.2) (layer "F.Cu") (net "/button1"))
 (segment (start 220 45.5) (end 220 38) (width 0.2) (layer "F.Cu") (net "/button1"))
 (segment (start 226.08 101.76) (end 226.751526 101.088474) (width 0.2) (layer "F.Cu") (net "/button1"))
 (segment (start 223.54 84.399899) (end 223.94 83.999899) (width 0.2) (layer "B.Cu") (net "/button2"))
 (segment (start 223.94 83.999899) (end 223.94 69.637056) (width 0.2) (layer "B.Cu") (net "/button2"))
 (segment (start 222.46 68.157056) (end 222.46 63.92) (width 0.2) (layer "B.Cu") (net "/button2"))
 (segment (start 223.54 101.76) (end 223.54 84.399899) (width 0.2) (layer "B.Cu") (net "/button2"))
 (segment (start 223.94 69.637056) (end 222.46 68.157056) (width 0.2) (layer "B.Cu") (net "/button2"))
 (segment (start 222.54 100.22) (end 222.54 83.42) (width 0.2) (layer "B.Cu") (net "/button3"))
 (segment (start 221 101.76) (end 222.54 100.22) (width 0.2) (layer "B.Cu") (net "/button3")))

